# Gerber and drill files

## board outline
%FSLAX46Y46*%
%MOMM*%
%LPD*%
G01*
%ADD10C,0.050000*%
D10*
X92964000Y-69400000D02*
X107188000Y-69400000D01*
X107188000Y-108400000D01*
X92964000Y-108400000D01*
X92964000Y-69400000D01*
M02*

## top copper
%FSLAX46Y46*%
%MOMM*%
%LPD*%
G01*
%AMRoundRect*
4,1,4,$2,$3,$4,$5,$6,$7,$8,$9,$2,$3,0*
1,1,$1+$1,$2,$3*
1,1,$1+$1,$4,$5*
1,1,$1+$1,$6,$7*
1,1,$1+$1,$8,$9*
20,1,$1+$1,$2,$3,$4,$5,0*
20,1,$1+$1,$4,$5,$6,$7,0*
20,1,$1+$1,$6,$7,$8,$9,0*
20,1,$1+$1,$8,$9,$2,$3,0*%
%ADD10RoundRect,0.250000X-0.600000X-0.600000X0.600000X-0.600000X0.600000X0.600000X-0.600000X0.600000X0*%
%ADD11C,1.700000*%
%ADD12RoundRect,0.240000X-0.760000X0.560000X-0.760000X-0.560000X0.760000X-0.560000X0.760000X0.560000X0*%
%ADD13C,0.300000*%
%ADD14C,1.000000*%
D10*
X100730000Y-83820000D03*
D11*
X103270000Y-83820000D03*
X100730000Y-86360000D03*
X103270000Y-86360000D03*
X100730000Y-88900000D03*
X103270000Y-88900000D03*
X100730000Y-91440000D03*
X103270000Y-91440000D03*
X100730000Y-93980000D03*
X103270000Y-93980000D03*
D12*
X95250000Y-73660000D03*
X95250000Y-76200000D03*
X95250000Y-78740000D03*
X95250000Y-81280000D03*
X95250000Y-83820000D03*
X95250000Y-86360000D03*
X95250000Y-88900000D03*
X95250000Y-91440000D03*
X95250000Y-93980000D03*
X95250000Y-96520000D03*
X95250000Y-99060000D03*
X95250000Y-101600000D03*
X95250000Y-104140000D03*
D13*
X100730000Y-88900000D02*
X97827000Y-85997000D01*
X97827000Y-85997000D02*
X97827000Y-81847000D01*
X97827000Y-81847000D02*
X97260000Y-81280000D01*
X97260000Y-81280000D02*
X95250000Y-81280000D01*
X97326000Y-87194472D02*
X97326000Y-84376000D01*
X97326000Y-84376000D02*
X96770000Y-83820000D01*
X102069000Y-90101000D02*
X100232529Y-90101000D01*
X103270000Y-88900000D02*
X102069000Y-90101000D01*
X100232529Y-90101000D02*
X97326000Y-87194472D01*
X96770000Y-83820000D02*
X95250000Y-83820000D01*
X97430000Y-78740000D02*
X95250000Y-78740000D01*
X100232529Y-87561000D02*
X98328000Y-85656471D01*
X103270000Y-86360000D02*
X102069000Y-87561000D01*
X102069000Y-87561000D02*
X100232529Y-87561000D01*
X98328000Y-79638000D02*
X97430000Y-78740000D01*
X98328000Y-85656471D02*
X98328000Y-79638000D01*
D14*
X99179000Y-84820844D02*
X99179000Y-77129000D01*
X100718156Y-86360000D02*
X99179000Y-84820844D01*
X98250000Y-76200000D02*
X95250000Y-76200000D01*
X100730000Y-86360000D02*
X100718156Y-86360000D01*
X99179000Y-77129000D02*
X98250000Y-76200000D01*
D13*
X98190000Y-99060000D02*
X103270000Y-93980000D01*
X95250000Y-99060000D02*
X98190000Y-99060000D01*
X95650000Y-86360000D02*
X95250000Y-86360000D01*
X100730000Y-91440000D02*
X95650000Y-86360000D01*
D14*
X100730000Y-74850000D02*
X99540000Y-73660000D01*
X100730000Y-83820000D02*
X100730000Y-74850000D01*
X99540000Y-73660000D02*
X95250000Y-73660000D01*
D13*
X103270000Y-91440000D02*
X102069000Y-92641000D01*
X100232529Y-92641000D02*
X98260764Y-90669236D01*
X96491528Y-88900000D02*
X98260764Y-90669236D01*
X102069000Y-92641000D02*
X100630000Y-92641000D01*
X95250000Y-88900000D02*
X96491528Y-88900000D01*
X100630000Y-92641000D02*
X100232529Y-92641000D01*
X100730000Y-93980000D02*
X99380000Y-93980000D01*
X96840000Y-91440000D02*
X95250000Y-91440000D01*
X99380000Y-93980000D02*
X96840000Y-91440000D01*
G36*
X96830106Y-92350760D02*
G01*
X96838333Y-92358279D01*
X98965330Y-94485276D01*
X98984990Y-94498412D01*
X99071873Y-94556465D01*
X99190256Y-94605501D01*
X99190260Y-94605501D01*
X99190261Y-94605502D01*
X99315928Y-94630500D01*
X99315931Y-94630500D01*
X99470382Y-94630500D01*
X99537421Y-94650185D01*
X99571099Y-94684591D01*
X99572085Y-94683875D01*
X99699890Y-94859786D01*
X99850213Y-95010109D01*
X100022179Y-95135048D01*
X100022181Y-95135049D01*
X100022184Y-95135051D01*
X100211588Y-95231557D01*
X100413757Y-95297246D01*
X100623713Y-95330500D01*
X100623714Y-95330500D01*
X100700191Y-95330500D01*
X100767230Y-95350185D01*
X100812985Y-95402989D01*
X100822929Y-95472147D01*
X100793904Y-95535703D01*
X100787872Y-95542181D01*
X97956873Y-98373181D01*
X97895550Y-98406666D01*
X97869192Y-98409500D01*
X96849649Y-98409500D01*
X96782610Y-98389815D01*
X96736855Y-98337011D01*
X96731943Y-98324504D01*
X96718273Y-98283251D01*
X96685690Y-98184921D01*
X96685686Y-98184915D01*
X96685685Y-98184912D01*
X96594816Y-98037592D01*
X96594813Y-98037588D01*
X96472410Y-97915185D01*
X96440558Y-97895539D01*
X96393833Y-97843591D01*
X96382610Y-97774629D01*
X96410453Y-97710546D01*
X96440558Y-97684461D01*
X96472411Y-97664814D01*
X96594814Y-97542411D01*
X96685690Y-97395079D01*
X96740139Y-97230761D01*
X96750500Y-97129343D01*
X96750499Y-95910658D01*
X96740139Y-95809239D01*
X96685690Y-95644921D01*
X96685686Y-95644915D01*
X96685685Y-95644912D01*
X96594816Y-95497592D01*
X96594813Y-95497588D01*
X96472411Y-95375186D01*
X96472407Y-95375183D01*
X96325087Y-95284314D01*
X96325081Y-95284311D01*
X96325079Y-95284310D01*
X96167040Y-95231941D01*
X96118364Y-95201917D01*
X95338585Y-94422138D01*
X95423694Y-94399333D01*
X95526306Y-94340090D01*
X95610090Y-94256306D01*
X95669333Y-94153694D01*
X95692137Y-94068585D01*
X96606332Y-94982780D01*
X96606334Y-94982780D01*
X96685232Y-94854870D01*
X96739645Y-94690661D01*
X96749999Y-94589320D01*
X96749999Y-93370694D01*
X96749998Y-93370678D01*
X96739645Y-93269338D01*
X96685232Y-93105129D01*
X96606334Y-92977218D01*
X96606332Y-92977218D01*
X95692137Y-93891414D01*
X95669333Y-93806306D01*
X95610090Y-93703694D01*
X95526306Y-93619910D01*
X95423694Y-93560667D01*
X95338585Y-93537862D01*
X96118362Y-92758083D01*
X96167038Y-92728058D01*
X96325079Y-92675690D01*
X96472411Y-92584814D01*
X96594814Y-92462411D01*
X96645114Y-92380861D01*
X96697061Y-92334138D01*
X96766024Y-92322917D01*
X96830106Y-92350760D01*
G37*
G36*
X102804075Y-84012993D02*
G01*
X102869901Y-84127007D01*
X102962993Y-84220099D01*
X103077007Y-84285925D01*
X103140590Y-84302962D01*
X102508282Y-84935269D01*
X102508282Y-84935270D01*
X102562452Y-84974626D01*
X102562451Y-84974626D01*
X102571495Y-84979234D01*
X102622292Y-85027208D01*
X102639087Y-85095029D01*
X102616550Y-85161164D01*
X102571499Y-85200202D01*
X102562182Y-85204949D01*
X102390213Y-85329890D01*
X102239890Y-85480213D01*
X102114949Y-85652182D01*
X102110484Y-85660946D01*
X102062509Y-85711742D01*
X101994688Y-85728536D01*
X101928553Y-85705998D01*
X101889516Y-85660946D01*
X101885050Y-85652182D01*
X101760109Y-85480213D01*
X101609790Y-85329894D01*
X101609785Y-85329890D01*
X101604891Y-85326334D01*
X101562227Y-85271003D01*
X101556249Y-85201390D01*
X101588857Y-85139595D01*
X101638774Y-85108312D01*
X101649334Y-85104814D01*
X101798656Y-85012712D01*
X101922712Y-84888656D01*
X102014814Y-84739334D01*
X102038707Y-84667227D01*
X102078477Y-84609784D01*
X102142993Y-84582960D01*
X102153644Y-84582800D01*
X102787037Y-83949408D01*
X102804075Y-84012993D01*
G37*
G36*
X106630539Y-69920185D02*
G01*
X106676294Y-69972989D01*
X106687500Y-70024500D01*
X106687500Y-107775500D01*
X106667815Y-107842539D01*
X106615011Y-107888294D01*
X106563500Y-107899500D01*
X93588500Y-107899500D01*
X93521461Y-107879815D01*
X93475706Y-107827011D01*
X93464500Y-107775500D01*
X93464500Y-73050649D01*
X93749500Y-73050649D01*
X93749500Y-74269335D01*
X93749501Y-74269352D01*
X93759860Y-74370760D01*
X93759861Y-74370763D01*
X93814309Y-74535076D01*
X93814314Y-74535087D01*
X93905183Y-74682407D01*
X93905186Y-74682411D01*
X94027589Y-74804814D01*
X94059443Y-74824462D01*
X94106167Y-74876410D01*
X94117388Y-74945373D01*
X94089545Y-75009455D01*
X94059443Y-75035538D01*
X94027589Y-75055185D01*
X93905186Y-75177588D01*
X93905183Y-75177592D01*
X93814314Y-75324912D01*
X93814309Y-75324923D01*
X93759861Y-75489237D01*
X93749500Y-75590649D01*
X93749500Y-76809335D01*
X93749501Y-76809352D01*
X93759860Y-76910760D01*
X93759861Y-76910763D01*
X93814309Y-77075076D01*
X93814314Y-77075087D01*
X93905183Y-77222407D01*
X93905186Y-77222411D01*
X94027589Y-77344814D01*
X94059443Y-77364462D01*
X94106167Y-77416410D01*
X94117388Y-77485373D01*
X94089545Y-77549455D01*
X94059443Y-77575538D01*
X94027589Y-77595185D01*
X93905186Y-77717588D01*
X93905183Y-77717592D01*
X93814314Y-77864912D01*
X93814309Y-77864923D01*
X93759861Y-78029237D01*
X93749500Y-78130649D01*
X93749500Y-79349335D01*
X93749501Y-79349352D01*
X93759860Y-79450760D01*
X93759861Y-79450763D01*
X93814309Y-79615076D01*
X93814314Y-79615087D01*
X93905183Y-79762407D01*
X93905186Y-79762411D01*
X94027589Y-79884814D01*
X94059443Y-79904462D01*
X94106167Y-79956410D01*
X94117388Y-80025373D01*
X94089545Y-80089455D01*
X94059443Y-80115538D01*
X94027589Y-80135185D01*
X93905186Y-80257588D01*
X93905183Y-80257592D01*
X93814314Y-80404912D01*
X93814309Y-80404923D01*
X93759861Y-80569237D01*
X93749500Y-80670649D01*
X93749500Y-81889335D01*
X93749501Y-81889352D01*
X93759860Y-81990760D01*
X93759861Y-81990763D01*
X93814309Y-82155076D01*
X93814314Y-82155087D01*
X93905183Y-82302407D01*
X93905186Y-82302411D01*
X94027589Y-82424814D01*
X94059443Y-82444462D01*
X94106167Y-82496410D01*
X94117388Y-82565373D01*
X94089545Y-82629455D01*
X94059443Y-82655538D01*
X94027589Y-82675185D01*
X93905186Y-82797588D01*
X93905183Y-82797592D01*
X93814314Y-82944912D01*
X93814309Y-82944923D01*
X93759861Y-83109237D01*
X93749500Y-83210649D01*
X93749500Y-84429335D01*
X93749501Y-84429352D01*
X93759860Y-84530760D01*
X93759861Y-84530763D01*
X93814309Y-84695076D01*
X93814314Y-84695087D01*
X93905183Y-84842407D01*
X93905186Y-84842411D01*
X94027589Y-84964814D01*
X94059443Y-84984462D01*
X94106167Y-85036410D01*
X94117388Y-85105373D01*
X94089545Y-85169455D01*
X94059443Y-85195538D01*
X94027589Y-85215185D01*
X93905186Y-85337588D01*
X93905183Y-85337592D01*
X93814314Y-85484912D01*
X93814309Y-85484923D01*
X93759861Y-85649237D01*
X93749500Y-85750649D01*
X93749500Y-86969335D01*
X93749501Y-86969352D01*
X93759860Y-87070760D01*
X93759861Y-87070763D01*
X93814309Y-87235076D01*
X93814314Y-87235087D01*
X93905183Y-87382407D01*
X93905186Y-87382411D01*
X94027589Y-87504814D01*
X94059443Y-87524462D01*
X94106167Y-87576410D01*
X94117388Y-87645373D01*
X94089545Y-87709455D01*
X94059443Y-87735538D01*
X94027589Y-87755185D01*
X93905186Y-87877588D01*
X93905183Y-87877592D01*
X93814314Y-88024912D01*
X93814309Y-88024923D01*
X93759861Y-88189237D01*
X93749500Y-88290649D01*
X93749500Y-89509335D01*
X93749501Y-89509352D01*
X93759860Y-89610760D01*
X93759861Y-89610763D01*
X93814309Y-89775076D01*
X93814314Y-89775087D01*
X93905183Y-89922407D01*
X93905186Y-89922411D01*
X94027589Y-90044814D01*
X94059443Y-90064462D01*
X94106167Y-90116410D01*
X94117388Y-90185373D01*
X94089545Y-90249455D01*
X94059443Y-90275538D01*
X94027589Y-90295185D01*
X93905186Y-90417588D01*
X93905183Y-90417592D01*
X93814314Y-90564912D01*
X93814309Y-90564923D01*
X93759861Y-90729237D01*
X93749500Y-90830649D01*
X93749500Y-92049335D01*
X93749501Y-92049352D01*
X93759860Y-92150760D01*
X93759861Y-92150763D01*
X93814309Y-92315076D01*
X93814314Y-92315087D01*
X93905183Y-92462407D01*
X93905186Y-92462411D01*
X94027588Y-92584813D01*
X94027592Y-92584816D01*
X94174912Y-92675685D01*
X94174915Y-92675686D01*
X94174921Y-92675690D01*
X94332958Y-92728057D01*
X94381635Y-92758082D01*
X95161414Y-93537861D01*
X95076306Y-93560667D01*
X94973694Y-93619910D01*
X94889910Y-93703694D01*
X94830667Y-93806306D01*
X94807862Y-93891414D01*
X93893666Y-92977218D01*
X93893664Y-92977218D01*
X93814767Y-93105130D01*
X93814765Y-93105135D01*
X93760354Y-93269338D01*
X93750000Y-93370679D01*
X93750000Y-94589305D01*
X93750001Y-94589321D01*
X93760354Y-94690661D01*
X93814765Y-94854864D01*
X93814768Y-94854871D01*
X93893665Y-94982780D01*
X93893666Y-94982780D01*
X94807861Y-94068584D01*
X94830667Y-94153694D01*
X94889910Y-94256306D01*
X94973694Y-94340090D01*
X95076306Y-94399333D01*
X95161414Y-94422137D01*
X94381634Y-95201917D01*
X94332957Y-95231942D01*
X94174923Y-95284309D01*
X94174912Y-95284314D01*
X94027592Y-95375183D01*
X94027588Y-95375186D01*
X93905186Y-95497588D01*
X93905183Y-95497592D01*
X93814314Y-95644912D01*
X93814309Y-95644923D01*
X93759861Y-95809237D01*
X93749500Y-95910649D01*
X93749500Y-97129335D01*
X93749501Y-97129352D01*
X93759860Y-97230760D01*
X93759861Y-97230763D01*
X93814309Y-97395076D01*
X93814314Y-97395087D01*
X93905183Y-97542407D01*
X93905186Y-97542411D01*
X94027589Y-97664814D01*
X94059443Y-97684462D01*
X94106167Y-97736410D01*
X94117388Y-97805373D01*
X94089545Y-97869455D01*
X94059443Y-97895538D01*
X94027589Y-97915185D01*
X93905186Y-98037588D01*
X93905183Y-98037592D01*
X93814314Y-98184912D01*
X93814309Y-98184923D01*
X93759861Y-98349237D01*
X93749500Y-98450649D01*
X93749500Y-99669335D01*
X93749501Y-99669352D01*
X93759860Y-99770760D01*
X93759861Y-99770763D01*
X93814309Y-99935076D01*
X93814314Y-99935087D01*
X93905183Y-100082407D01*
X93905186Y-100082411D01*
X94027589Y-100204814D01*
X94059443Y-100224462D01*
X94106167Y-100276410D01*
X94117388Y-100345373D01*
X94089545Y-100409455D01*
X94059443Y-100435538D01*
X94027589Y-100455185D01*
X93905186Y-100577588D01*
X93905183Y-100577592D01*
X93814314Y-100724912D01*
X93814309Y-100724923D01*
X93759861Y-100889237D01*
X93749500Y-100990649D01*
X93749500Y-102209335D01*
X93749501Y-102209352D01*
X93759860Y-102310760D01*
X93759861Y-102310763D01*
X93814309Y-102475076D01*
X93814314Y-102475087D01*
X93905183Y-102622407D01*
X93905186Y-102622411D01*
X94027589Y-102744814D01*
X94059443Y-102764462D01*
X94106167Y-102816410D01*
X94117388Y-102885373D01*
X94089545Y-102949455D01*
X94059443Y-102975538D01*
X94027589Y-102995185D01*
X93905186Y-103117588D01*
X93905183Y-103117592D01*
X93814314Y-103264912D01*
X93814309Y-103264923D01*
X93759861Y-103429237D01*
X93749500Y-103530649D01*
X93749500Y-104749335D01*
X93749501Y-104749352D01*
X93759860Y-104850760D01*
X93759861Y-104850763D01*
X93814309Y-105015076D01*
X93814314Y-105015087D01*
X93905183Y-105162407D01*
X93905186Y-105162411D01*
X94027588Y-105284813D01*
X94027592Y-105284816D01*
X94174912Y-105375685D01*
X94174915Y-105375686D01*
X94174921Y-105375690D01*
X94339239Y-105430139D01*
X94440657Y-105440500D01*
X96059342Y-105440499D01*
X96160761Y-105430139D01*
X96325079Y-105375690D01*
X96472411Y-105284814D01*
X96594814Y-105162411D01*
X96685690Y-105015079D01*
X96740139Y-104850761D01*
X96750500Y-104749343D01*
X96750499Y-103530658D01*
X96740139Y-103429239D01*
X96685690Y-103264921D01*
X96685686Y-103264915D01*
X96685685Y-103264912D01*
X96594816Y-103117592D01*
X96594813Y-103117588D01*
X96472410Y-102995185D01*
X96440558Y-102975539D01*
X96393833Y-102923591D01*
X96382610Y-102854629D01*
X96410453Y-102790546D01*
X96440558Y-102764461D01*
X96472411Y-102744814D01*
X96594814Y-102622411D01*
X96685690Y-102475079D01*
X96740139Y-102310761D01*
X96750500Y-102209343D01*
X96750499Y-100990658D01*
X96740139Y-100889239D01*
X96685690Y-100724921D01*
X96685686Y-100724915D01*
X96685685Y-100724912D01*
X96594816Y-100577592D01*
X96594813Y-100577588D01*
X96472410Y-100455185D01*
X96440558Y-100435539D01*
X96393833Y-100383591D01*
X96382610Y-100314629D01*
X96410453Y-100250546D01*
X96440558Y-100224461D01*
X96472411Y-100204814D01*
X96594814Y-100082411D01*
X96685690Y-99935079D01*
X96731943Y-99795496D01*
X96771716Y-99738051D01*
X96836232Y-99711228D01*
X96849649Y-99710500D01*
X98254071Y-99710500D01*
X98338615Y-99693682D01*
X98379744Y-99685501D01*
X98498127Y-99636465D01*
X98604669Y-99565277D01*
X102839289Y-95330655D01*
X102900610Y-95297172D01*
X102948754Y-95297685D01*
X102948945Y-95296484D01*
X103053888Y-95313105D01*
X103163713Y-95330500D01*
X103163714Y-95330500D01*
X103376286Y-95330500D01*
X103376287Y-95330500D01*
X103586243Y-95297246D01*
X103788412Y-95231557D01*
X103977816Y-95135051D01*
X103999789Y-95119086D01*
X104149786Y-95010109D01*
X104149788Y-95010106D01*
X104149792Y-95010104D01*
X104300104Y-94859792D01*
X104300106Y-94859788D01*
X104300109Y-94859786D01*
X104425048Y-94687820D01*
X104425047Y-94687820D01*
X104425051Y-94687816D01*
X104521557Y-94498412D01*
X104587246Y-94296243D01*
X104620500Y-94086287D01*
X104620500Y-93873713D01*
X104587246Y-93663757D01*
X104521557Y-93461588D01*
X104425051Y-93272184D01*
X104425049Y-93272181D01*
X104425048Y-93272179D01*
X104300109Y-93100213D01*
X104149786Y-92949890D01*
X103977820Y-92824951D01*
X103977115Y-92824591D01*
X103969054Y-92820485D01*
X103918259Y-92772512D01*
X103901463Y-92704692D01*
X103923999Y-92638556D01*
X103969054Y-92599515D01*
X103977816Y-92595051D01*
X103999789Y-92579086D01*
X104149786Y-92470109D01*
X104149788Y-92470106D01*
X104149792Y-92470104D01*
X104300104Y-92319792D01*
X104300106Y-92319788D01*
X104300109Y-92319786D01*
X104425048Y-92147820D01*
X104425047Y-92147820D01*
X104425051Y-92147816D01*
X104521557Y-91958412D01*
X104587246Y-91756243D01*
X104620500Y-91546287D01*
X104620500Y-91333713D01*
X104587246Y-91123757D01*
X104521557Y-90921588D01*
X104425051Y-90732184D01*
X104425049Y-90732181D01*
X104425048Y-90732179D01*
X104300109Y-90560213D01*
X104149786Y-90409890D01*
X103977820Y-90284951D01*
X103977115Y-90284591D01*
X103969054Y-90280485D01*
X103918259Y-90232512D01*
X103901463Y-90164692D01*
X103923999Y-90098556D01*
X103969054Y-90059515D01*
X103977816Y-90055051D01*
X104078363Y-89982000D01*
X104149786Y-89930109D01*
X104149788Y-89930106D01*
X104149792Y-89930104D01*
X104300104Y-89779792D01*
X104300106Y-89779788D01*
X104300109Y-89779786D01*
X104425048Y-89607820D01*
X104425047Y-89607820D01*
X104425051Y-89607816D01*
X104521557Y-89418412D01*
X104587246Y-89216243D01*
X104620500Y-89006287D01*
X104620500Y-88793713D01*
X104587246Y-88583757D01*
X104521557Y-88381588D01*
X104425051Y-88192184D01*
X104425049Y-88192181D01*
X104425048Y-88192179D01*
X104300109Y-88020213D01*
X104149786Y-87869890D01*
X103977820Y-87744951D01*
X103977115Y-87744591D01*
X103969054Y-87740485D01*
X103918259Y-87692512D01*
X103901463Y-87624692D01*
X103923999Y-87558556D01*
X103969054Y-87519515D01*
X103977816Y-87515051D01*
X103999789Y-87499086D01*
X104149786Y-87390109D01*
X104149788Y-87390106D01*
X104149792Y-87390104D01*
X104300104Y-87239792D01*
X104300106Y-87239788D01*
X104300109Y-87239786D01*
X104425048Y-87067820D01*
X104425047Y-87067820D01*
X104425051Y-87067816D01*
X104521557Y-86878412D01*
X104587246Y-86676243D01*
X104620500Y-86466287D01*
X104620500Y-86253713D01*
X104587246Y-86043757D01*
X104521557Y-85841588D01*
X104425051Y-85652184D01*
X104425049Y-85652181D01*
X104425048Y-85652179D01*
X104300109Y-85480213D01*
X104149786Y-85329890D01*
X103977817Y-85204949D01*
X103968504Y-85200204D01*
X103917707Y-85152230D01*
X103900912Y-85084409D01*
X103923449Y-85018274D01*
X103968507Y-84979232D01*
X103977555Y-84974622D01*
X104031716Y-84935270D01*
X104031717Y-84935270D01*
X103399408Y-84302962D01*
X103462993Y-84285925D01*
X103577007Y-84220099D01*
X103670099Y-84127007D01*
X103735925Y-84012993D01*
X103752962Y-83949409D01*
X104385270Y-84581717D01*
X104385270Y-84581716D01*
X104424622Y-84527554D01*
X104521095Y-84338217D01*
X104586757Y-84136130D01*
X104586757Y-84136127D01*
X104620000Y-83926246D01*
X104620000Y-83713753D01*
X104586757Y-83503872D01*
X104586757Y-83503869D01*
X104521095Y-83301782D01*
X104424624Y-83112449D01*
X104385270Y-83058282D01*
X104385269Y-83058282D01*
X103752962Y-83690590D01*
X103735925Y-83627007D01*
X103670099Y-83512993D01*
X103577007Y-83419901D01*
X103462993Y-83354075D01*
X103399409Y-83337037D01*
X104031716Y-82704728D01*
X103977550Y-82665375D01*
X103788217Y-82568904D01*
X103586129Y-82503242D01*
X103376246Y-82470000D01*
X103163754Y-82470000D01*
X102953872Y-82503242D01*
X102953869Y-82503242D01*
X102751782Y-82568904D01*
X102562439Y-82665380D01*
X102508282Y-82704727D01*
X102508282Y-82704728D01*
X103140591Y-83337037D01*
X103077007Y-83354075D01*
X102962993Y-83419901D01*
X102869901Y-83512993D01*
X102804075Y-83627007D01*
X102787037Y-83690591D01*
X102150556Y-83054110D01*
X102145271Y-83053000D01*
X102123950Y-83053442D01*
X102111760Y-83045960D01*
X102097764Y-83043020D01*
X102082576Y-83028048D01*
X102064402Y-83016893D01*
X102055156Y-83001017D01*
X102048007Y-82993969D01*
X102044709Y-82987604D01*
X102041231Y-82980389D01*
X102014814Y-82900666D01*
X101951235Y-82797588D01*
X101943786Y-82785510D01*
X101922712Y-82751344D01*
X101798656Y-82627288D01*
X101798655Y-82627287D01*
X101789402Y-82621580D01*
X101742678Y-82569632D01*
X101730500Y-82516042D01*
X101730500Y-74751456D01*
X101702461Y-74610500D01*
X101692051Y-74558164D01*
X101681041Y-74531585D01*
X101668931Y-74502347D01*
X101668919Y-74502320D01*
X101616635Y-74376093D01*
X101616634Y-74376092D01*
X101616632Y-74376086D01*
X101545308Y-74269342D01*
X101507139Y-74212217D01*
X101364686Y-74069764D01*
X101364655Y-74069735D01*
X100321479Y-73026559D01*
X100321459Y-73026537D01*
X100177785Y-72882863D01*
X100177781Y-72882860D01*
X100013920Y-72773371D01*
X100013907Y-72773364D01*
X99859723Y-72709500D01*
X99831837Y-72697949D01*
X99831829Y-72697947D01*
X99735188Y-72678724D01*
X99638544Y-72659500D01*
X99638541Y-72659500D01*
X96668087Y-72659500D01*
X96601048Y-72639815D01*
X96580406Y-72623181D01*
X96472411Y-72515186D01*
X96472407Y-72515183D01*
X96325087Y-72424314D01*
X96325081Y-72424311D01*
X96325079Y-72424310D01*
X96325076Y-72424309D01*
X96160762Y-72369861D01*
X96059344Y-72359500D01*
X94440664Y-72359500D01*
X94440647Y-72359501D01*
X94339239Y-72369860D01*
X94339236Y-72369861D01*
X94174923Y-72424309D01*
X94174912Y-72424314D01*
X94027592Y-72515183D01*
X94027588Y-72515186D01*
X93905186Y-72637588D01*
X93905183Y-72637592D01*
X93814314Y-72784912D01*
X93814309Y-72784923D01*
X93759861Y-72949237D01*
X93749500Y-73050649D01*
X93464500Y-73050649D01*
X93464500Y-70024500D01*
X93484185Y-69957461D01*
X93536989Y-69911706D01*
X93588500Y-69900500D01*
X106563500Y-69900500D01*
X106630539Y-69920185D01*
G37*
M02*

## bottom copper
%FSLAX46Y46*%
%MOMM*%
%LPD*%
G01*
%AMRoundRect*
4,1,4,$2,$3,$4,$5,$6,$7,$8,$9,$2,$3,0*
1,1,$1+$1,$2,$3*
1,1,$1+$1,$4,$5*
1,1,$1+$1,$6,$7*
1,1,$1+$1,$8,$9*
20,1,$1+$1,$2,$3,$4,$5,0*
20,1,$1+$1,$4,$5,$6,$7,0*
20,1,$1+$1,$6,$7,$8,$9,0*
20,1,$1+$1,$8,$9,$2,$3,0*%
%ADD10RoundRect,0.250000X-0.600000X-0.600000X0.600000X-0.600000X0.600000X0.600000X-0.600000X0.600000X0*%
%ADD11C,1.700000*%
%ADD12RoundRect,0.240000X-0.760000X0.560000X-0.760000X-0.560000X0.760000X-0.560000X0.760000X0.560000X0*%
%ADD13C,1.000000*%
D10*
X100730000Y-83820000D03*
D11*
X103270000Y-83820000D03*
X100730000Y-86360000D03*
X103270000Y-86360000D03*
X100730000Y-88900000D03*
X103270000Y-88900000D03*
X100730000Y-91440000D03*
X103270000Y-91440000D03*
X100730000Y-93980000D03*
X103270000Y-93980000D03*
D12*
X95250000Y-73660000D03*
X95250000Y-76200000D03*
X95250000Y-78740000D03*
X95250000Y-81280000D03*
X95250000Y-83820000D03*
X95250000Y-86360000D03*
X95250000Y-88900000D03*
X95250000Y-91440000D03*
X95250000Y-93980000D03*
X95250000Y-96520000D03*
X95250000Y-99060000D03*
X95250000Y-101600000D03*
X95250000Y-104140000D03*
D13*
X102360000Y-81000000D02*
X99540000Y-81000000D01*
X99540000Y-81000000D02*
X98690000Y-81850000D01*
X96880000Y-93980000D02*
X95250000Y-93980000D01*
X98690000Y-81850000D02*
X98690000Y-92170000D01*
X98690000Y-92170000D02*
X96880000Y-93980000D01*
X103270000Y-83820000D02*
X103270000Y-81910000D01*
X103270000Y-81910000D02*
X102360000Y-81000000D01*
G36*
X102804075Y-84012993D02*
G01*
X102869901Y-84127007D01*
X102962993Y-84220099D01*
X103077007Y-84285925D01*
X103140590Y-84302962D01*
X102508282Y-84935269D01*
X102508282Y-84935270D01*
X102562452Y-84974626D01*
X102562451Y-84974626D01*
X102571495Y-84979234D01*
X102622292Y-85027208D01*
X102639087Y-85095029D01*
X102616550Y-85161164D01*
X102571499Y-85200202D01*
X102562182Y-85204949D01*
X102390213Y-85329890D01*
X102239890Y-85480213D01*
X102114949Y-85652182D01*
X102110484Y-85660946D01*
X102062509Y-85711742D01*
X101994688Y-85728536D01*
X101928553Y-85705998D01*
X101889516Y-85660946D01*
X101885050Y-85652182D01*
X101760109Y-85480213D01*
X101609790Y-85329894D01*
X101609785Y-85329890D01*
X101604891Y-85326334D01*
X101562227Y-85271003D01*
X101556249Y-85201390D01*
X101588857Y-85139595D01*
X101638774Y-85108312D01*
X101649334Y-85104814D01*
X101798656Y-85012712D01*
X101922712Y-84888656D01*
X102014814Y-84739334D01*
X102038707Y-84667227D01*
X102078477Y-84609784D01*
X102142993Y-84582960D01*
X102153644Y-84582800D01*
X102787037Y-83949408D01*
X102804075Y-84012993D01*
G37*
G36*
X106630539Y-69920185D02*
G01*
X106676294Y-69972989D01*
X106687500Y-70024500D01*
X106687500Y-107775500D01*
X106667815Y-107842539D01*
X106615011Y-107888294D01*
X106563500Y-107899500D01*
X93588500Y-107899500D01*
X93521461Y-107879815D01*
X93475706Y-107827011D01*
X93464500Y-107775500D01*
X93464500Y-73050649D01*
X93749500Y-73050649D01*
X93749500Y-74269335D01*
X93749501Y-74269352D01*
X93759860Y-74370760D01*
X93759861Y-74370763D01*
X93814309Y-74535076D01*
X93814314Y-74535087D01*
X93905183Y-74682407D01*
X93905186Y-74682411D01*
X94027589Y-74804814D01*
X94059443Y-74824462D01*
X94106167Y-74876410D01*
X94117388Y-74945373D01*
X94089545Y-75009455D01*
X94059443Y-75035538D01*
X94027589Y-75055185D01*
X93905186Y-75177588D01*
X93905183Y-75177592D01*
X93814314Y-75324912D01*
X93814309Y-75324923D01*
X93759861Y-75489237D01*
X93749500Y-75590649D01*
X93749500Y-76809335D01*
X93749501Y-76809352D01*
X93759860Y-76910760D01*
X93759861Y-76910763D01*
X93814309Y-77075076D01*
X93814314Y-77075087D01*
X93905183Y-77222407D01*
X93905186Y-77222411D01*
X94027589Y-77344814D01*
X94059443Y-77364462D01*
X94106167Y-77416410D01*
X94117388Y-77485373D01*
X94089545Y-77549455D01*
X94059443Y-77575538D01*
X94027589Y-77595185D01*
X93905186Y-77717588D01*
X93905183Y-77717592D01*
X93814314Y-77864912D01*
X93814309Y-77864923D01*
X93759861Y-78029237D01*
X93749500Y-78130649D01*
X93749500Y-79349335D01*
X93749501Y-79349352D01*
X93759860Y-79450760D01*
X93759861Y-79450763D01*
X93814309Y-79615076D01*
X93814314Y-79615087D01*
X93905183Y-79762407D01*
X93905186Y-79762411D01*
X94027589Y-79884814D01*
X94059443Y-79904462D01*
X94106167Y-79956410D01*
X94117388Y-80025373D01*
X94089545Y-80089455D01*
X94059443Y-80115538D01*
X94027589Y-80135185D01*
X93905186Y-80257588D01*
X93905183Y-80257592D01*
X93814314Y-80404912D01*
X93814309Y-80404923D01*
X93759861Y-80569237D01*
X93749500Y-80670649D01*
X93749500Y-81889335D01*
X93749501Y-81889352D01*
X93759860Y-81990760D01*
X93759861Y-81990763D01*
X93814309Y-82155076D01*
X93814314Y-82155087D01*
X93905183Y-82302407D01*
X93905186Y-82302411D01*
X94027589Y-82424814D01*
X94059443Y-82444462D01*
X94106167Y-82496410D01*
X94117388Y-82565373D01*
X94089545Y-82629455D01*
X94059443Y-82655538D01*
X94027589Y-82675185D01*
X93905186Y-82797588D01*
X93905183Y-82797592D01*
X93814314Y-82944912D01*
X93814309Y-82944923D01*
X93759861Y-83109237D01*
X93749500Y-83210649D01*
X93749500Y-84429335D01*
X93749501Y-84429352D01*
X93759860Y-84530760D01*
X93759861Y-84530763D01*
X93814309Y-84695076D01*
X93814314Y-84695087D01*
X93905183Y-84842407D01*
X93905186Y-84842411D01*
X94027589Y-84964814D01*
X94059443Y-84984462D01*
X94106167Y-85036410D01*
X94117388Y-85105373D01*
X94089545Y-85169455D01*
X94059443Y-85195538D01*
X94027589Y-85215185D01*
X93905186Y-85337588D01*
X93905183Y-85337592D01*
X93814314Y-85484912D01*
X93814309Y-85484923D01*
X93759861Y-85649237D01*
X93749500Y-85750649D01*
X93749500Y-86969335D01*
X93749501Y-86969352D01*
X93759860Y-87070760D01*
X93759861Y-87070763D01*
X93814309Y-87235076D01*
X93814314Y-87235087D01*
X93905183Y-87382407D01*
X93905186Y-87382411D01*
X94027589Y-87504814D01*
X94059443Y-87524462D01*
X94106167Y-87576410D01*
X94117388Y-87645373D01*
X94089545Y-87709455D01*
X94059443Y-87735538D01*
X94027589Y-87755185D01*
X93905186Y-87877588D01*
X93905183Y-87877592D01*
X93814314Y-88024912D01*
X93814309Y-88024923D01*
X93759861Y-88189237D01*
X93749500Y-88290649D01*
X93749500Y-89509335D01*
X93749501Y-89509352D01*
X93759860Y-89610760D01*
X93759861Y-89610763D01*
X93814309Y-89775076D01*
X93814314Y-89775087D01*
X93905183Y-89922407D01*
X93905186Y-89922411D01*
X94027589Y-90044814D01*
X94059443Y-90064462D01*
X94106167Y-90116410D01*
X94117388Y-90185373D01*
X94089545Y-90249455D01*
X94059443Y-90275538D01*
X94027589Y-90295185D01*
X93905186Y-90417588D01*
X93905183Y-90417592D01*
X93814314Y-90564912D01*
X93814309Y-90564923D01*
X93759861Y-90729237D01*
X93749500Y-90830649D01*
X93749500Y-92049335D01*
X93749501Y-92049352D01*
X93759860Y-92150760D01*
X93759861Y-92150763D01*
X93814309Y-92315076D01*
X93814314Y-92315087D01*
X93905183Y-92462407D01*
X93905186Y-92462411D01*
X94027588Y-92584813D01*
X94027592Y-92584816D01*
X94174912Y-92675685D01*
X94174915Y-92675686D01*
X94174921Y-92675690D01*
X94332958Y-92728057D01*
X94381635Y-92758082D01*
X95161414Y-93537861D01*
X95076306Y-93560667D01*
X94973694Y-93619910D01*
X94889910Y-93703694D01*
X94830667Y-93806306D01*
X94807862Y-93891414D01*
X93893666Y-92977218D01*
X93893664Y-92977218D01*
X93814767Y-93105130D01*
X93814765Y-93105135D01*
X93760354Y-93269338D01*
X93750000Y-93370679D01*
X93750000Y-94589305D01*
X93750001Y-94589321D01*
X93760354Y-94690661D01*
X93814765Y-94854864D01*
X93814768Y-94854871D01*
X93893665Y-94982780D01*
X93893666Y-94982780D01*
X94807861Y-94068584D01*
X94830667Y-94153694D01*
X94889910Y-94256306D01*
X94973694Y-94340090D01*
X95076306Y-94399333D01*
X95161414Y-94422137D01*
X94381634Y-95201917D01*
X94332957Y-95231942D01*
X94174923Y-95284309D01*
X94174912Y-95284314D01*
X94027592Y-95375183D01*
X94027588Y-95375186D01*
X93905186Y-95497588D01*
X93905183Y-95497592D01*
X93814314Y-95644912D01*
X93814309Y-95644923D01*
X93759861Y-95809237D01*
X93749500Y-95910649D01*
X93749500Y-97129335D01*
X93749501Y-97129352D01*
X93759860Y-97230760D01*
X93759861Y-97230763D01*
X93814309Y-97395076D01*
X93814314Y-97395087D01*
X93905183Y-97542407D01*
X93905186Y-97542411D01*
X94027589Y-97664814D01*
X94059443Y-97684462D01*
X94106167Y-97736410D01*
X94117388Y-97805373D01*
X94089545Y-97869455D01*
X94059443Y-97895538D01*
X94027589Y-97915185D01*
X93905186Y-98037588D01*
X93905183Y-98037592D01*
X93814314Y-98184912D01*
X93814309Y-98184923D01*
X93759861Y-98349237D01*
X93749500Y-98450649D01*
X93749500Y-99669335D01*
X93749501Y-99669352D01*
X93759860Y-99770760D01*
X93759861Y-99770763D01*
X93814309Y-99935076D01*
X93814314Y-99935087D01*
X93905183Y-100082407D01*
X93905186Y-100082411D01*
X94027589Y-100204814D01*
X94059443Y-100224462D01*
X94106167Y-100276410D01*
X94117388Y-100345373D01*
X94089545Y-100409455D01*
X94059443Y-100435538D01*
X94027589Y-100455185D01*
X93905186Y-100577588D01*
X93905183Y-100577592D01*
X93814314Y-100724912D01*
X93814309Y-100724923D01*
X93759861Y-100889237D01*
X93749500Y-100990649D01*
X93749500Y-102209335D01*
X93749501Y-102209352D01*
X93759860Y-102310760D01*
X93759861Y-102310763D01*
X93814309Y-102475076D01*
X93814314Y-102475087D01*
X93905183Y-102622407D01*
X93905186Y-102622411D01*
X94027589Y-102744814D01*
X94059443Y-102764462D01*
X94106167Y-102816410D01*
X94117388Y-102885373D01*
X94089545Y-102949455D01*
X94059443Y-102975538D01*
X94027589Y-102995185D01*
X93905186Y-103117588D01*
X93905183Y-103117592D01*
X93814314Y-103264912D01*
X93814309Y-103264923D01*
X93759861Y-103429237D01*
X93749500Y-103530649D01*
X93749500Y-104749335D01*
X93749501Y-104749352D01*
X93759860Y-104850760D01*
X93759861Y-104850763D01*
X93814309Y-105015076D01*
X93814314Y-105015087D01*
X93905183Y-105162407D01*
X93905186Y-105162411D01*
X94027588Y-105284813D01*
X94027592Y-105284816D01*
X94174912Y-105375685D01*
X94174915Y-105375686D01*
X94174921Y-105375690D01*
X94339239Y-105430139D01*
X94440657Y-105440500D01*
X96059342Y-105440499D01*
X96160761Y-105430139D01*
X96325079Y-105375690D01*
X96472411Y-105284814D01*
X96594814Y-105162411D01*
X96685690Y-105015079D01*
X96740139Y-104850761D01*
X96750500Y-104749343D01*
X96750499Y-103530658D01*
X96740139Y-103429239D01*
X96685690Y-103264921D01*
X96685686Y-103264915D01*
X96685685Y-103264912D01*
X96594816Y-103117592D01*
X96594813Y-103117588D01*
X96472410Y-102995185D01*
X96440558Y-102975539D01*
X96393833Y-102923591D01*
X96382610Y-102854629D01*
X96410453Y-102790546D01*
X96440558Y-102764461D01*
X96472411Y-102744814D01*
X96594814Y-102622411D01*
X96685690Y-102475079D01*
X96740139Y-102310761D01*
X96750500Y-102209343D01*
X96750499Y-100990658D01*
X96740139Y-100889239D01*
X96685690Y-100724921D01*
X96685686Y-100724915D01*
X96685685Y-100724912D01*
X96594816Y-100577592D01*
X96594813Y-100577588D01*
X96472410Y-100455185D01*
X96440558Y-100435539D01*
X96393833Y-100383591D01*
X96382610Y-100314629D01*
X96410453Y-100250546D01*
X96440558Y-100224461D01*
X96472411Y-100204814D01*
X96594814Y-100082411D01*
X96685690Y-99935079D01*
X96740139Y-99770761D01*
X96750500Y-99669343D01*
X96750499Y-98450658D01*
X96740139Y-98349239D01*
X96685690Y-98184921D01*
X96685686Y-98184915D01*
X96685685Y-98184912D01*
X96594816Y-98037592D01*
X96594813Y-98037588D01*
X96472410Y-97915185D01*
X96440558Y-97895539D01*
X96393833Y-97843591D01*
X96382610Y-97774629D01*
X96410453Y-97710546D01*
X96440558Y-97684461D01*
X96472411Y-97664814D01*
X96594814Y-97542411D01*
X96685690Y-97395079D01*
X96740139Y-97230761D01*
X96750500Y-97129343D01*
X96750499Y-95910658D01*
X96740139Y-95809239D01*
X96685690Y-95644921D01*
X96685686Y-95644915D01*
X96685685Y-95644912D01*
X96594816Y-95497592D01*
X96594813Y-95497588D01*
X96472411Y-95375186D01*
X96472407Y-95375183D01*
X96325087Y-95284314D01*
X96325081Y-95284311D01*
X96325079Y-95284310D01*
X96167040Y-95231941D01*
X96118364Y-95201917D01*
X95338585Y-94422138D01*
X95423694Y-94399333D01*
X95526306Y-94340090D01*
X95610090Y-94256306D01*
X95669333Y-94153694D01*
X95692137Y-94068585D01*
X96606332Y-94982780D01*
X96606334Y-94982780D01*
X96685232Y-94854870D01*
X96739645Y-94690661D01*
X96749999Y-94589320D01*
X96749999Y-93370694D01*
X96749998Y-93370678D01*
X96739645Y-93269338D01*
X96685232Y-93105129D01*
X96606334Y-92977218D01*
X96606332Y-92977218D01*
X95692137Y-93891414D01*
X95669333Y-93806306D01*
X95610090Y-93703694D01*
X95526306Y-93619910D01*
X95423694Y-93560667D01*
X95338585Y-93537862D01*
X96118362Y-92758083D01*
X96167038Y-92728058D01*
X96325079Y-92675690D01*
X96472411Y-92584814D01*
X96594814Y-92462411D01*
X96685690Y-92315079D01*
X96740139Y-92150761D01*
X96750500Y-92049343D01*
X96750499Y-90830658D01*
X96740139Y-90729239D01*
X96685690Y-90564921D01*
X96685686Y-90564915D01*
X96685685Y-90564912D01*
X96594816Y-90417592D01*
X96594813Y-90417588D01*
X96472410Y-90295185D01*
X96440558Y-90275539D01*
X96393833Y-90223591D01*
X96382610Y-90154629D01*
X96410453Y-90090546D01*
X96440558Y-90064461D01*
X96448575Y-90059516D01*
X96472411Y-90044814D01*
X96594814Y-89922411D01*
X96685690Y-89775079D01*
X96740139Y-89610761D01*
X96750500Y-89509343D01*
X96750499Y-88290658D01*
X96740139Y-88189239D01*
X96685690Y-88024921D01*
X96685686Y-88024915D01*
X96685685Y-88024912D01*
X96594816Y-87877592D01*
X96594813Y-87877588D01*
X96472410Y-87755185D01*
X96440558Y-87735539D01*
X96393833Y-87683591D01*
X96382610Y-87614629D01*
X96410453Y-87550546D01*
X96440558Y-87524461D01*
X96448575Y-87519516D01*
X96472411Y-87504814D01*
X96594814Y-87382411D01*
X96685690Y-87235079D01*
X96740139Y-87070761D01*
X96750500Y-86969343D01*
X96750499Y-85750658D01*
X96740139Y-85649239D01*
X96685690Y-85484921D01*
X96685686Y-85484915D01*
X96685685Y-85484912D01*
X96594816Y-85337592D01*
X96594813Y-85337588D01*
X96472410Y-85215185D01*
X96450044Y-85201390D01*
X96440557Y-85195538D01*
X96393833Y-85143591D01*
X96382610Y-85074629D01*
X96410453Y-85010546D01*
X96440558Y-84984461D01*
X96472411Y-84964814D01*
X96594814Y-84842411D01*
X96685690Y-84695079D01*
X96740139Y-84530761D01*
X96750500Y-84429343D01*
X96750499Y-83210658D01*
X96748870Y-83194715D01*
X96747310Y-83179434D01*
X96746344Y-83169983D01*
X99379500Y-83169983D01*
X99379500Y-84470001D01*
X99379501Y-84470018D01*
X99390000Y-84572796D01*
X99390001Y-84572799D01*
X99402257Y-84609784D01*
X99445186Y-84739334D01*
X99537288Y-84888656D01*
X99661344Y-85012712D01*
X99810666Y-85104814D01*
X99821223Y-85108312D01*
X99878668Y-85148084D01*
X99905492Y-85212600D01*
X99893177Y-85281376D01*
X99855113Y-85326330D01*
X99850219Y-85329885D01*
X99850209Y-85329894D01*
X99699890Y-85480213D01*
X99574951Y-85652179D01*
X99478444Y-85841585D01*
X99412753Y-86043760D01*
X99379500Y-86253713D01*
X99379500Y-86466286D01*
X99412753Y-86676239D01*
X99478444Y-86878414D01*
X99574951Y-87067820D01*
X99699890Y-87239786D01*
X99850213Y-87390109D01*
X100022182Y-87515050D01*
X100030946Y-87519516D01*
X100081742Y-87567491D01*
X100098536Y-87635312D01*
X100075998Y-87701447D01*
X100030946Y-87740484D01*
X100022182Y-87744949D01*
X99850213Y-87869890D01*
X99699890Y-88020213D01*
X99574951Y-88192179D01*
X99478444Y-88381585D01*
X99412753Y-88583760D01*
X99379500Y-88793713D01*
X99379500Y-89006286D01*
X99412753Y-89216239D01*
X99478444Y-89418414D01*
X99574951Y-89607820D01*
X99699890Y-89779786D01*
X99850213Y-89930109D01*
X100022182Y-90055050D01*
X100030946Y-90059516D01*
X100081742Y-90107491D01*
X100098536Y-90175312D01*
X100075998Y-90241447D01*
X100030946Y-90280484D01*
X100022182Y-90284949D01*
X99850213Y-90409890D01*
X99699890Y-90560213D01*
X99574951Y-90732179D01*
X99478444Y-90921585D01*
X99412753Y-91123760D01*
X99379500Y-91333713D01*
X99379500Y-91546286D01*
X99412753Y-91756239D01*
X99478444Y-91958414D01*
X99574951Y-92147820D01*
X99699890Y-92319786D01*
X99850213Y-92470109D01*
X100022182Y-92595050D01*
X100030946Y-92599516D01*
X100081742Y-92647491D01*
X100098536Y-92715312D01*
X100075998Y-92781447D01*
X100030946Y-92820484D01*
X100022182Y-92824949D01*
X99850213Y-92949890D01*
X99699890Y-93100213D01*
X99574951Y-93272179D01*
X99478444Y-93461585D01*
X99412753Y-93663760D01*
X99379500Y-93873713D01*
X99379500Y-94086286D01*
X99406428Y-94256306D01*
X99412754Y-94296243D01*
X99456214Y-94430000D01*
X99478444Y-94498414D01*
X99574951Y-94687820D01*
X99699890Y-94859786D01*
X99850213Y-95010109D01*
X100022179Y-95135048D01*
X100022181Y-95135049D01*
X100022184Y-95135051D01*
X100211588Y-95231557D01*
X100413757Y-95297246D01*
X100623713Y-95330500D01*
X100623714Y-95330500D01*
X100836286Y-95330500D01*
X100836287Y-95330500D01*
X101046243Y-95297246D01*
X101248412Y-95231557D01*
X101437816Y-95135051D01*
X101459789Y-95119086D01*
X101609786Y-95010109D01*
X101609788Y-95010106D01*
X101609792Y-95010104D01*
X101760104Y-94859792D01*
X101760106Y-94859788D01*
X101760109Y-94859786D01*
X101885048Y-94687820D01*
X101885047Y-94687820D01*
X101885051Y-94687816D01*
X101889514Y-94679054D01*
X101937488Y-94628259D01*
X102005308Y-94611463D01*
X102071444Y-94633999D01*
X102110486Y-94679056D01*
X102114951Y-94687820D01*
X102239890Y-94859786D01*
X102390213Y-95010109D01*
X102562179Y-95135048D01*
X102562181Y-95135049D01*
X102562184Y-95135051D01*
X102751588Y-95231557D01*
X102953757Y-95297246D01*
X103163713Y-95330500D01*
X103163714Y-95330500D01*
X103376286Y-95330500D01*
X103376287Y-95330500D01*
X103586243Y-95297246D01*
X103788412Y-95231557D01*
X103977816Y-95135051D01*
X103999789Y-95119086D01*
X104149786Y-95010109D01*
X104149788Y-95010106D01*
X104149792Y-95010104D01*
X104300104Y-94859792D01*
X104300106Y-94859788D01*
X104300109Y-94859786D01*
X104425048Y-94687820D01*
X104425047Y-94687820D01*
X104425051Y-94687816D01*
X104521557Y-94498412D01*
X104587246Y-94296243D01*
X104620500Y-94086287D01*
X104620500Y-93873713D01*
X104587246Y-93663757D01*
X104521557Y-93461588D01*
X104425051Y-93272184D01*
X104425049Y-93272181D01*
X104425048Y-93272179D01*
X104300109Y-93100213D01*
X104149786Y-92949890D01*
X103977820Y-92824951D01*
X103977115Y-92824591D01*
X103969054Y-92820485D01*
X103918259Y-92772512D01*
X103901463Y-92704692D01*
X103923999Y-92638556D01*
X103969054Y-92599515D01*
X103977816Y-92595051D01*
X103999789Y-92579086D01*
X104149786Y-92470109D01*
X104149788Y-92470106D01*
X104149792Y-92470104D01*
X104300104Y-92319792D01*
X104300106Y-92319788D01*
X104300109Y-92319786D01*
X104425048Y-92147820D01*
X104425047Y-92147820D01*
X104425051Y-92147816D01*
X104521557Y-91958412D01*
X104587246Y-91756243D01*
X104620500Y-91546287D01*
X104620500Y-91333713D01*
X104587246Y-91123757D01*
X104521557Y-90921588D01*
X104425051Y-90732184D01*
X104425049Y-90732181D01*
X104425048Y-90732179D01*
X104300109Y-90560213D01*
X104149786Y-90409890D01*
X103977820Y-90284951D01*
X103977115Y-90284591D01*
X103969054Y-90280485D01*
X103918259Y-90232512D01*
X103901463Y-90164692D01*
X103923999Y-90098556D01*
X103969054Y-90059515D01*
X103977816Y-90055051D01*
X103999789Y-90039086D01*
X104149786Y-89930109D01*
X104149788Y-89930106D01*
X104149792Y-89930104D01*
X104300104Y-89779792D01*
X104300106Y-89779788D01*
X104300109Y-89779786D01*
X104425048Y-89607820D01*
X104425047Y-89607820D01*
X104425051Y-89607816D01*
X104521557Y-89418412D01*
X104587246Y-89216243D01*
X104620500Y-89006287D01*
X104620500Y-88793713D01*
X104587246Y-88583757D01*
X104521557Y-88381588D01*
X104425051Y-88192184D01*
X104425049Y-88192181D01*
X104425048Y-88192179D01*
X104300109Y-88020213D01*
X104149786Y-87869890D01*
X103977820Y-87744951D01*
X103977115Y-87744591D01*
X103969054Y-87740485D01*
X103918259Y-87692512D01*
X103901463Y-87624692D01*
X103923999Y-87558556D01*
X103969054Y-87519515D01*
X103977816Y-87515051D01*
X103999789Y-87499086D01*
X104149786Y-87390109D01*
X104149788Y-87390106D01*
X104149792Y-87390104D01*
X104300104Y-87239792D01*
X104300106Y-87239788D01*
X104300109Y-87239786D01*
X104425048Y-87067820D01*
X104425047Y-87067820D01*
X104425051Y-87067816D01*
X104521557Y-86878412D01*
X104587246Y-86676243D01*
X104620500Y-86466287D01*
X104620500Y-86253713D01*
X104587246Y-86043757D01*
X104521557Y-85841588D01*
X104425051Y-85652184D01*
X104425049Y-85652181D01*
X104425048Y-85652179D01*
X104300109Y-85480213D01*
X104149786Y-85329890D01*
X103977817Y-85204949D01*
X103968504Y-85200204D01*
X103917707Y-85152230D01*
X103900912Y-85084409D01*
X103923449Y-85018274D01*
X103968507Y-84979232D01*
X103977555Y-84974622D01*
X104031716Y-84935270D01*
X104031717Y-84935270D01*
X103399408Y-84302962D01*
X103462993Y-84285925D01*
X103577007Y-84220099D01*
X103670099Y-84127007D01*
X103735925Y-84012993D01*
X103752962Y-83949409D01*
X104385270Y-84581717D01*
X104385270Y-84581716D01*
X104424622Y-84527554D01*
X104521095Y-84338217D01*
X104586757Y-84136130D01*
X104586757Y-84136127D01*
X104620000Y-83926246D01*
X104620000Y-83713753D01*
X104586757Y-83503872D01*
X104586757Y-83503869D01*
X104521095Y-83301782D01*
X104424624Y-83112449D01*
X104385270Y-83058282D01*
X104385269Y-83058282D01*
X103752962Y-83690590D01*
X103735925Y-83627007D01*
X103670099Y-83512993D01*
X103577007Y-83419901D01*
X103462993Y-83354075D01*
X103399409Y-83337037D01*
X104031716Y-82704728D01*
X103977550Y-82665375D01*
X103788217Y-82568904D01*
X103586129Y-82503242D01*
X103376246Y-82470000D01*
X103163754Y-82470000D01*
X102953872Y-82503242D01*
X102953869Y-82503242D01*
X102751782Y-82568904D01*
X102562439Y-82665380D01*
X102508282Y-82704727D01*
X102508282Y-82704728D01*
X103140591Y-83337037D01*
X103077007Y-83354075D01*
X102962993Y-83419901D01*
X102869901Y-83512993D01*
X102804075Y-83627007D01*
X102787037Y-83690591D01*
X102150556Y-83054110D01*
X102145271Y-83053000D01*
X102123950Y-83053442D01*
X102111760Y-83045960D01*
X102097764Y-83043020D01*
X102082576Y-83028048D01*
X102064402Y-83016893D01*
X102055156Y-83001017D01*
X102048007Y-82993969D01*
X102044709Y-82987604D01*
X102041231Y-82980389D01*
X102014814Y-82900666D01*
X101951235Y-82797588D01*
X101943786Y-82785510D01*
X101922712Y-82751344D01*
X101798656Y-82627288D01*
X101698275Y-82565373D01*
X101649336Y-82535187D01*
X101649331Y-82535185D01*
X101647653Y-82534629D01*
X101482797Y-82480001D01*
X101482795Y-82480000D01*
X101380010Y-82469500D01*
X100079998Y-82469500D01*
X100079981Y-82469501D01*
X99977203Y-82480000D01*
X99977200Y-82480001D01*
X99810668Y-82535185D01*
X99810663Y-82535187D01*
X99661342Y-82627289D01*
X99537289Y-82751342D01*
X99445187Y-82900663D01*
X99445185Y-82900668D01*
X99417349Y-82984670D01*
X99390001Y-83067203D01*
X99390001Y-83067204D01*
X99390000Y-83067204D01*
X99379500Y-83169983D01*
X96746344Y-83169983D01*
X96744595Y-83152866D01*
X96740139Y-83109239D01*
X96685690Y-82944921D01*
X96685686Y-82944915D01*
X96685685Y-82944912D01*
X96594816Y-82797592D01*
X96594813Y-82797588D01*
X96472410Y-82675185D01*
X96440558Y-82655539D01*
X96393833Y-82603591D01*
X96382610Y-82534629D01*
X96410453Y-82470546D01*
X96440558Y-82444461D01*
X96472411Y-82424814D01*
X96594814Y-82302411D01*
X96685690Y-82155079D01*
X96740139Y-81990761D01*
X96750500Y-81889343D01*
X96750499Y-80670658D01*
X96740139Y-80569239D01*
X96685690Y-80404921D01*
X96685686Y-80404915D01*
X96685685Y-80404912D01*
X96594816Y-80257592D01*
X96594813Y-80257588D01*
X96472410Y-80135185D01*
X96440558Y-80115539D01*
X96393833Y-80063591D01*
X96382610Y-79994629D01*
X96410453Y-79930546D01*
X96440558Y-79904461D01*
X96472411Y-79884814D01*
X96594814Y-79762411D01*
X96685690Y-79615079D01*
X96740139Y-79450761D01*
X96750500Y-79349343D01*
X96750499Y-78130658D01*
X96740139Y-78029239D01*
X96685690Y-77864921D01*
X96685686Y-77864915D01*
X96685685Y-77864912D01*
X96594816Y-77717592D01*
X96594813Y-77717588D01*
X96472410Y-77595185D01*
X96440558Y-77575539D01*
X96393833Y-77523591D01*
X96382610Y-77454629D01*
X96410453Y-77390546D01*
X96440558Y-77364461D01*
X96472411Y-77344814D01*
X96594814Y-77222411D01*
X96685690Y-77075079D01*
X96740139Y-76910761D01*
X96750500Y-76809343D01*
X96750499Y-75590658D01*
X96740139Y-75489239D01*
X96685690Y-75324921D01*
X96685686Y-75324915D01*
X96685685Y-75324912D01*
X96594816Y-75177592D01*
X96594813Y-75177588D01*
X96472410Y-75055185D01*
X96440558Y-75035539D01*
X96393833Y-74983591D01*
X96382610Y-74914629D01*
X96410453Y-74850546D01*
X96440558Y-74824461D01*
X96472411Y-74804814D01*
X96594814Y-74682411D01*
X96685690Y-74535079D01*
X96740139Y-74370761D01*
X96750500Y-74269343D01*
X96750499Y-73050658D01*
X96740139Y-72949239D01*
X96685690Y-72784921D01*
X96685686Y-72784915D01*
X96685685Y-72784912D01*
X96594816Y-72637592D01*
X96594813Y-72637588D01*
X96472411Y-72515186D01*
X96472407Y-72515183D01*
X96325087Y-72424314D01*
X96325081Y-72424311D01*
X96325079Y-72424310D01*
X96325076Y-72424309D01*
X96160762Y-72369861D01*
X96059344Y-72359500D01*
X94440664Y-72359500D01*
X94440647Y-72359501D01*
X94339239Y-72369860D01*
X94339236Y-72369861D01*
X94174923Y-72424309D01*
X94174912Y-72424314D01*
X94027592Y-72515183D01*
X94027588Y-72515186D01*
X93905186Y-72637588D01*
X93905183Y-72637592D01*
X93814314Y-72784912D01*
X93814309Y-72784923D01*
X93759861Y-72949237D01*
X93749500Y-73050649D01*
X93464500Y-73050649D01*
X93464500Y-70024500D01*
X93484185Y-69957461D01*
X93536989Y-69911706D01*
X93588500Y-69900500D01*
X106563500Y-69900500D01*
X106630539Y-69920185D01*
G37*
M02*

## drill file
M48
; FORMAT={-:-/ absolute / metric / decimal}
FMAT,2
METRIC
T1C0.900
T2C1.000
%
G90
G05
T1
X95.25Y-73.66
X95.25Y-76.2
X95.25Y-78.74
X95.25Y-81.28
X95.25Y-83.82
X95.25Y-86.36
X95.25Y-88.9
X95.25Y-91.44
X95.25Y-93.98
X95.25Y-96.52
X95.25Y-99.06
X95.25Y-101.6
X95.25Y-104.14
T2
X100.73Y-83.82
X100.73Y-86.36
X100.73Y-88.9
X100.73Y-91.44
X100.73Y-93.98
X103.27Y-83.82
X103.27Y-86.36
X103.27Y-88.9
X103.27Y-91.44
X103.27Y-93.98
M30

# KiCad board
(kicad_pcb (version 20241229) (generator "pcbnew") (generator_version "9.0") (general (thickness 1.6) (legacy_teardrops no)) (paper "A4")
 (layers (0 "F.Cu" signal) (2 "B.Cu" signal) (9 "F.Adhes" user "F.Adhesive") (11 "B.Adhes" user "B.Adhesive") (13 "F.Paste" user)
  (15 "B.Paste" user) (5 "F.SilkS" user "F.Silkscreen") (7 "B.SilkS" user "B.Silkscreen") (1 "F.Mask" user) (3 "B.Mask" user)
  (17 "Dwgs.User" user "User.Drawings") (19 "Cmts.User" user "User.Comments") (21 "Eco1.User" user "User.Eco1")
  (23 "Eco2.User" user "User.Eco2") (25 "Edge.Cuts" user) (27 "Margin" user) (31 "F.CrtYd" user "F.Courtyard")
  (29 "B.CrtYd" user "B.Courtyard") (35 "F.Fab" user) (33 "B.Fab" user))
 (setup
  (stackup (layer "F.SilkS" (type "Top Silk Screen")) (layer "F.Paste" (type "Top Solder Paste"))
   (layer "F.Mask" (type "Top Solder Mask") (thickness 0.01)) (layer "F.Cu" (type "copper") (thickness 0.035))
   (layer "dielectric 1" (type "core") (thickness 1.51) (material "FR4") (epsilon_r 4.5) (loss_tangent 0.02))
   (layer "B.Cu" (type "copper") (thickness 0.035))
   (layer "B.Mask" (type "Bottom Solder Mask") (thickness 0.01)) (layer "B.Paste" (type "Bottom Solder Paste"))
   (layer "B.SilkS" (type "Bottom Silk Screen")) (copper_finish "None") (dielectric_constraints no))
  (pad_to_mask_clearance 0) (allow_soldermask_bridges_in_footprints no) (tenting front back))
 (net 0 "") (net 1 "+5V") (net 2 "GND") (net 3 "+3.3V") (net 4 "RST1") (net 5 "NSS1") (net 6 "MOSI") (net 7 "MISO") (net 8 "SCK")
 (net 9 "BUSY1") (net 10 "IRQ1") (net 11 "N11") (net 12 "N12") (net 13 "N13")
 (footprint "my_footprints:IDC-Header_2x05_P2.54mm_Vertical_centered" (layer "F.Cu") (at 102 88.9)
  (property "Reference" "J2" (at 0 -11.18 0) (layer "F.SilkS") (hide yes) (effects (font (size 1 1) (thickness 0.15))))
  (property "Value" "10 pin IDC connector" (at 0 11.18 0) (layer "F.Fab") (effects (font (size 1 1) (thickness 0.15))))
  (pad "1" thru_hole roundrect (at -1.27 -5.08) (size 1.7 1.7) (drill 1) (layers "*.Cu" "*.Mask") (remove_unused_layers no)
   (roundrect_rratio 0.147059) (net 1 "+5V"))
  (pad "2" thru_hole circle (at 1.27 -5.08) (size 1.7 1.7) (drill 1) (layers "*.Cu" "*.Mask") (remove_unused_layers no) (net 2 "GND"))
  (pad "3" thru_hole circle (at -1.27 -2.54) (size 1.7 1.7) (drill 1) (layers "*.Cu" "*.Mask") (remove_unused_layers no) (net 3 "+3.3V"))
  (pad "4" thru_hole circle (at 1.27 -2.54) (size 1.7 1.7) (drill 1) (layers "*.Cu" "*.Mask") (remove_unused_layers no) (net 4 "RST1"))
  (pad "5" thru_hole circle (at -1.27 0) (size 1.7 1.7) (drill 1) (layers "*.Cu" "*.Mask") (remove_unused_layers no) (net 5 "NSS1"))
  (pad "6" thru_hole circle (at 1.27 0) (size 1.7 1.7) (drill 1) (layers "*.Cu" "*.Mask") (remove_unused_layers no) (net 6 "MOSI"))
  (pad "7" thru_hole circle (at -1.27 2.54) (size 1.7 1.7) (drill 1) (layers "*.Cu" "*.Mask") (remove_unused_layers no) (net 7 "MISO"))
  (pad "8" thru_hole circle (at 1.27 2.54) (size 1.7 1.7) (drill 1) (layers "*.Cu" "*.Mask") (remove_unused_layers no) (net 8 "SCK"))
  (pad "9" thru_hole circle (at -1.27 5.08) (size 1.7 1.7) (drill 1) (layers "*.Cu" "*.Mask") (remove_unused_layers no) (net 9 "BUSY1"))
  (pad "10" thru_hole circle (at 1.27 5.08) (size 1.7 1.7) (drill 1) (layers "*.Cu" "*.Mask") (remove_unused_layers no) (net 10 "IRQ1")))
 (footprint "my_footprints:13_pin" (layer "F.Cu") (at 95.25 88.9 -90)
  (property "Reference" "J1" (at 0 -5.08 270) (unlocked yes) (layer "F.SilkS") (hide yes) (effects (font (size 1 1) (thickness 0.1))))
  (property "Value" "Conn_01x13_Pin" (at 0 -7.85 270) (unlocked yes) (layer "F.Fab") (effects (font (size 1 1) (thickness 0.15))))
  (pad "1" thru_hole roundrect (at -15.24 0 270) (size 1.6 2) (drill 0.9) (layers "*.Cu" "*.Mask") (remove_unused_layers no)
   (roundrect_rratio 0.15) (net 1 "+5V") (thermal_bridge_angle 45))
  (pad "2" thru_hole roundrect (at -12.7 0 270) (size 1.6 2) (drill 0.9) (layers "*.Cu" "*.Mask") (remove_unused_layers no)
   (roundrect_rratio 0.15) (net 3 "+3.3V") (thermal_bridge_angle 45))
  (pad "3" thru_hole roundrect (at -10.16 0 270) (size 1.6 2) (drill 0.9) (layers "*.Cu" "*.Mask") (remove_unused_layers no)
   (roundrect_rratio 0.15) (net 4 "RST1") (thermal_bridge_angle 45))
  (pad "4" thru_hole roundrect (at -7.62 0 270) (size 1.6 2) (drill 0.9) (layers "*.Cu" "*.Mask") (remove_unused_layers no)
   (roundrect_rratio 0.15) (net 5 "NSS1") (thermal_bridge_angle 45))
  (pad "5" thru_hole roundrect (at -5.08 0 270) (size 1.6 2) (drill 0.9) (layers "*.Cu" "*.Mask") (remove_unused_layers no)
   (roundrect_rratio 0.15) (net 6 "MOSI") (thermal_bridge_angle 45))
  (pad "6" thru_hole roundrect (at -2.54 0 270) (size 1.6 2) (drill 0.9) (layers "*.Cu" "*.Mask") (remove_unused_layers no)
   (roundrect_rratio 0.15) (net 7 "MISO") (thermal_bridge_angle 45))
  (pad "7" thru_hole roundrect (at 0 0 270) (size 1.6 2) (drill 0.9) (layers "*.Cu" "*.Mask") (remove_unused_layers no)
   (roundrect_rratio 0.15) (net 8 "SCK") (thermal_bridge_angle 45))
  (pad "8" thru_hole roundrect (at 2.54 0 270) (size 1.6 2) (drill 0.9) (layers "*.Cu" "*.Mask") (remove_unused_layers no)
   (roundrect_rratio 0.15) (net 9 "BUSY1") (thermal_bridge_angle 45))
  (pad "9" thru_hole roundrect (at 5.08 0 270) (size 1.6 2) (drill 0.9) (layers "*.Cu" "*.Mask") (remove_unused_layers no)
   (roundrect_rratio 0.15) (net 2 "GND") (thermal_bridge_angle 45))
  (pad "10" thru_hole roundrect (at 7.62 0 270) (size 1.6 2) (drill 0.9) (layers "*.Cu" "*.Mask") (remove_unused_layers no)
   (roundrect_rratio 0.15) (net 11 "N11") (thermal_bridge_angle 45))
  (pad "11" thru_hole roundrect (at 10.16 0 270) (size 1.6 2) (drill 0.9) (layers "*.Cu" "*.Mask") (remove_unused_layers no)
   (roundrect_rratio 0.15) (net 10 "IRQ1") (thermal_bridge_angle 45))
  (pad "12" thru_hole roundrect (at 12.7 0 270) (size 1.6 2) (drill 0.9) (layers "*.Cu" "*.Mask") (remove_unused_layers no)
   (roundrect_rratio 0.15) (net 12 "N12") (thermal_bridge_angle 45))
  (pad "13" thru_hole roundrect (at 15.24 0 270) (size 1.6 2) (drill 0.9) (layers "*.Cu" "*.Mask") (remove_unused_layers no)
   (roundrect_rratio 0.15) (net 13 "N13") (thermal_bridge_angle 45)))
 (gr_rect (start 92.964 69.4) (end 107.188 108.4) (stroke (width 0.05) (type solid)) (fill no) (layer "Edge.Cuts"))
 (segment (start 100.73 88.9) (end 97.827 85.997) (width 0.3) (layer "F.Cu") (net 5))
 (segment (start 97.827 85.997) (end 97.827 81.847) (width 0.3) (layer "F.Cu") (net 5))
 (segment (start 97.827 81.847) (end 97.26 81.28) (width 0.3) (layer "F.Cu") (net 5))
 (segment (start 97.26 81.28) (end 95.25 81.28) (width 0.3) (layer "F.Cu") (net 5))
 (segment (start 97.326 87.194472) (end 97.326 84.376) (width 0.3) (layer "F.Cu") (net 6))
 (segment (start 97.326 84.376) (end 96.77 83.82) (width 0.3) (layer "F.Cu") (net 6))
 (segment (start 102.069 90.101) (end 100.232529 90.101) (width 0.3) (layer "F.Cu") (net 6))
 (segment (start 103.27 88.9) (end 102.069 90.101) (width 0.3) (layer "F.Cu") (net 6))
 (segment (start 100.232529 90.101) (end 97.326 87.194472) (width 0.3) (layer "F.Cu") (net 6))
 (segment (start 96.77 83.82) (end 95.25 83.82) (width 0.3) (layer "F.Cu") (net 6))
 (segment (start 97.43 78.74) (end 95.25 78.74) (width 0.3) (layer "F.Cu") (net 4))
 (segment (start 100.232529 87.561) (end 98.328 85.656471) (width 0.3) (layer "F.Cu") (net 4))
 (segment (start 103.27 86.36) (end 102.069 87.561) (width 0.3) (layer "F.Cu") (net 4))
 (segment (start 102.069 87.561) (end 100.232529 87.561) (width 0.3) (layer "F.Cu") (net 4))
 (segment (start 98.328 79.638) (end 97.43 78.74) (width 0.3) (layer "F.Cu") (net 4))
 (segment (start 98.328 85.656471) (end 98.328 79.638) (width 0.3) (layer "F.Cu") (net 4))
 (segment (start 99.179 84.820844) (end 99.179 77.129) (width 1) (layer "F.Cu") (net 3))
 (segment (start 100.718156 86.36) (end 99.179 84.820844) (width 1) (layer "F.Cu") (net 3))
 (segment (start 98.25 76.2) (end 95.25 76.2) (width 1) (layer "F.Cu") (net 3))
 (segment (start 100.73 86.36) (end 100.718156 86.36) (width 1) (layer "F.Cu") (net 3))
 (segment (start 99.179 77.129) (end 98.25 76.2) (width 1) (layer "F.Cu") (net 3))
 (segment (start 98.19 99.06) (end 103.27 93.98) (width 0.3) (layer "F.Cu") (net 10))
 (segment (start 95.25 99.06) (end 98.19 99.06) (width 0.3) (layer "F.Cu") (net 10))
 (segment (start 95.65 86.36) (end 95.25 86.36) (width 0.3) (layer "F.Cu") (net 7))
 (segment (start 100.73 91.44) (end 95.65 86.36) (width 0.3) (layer "F.Cu") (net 7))
 (segment (start 100.73 74.85) (end 99.54 73.66) (width 1) (layer "F.Cu") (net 1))
 (segment (start 100.73 83.82) (end 100.73 74.85) (width 1) (layer "F.Cu") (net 1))
 (segment (start 99.54 73.66) (end 95.25 73.66) (width 1) (layer "F.Cu") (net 1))
 (segment (start 102.36 81) (end 99.54 81) (width 1) (layer "B.Cu") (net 2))
 (segment (start 99.54 81) (end 98.69 81.85) (width 1) (layer "B.Cu") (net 2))
 (segment (start 96.88 93.98) (end 95.25 93.98) (width 1) (layer "B.Cu") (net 2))
 (segment (start 98.69 81.85) (end 98.69 92.17) (width 1) (layer "B.Cu") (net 2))
 (segment (start 98.69 92.17) (end 96.88 93.98) (width 1) (layer "B.Cu") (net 2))
 (segment (start 103.27 83.82) (end 103.27 81.91) (width 1) (layer "B.Cu") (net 2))
 (segment (start 103.27 81.91) (end 102.36 81) (width 1) (layer "B.Cu") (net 2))
 (segment (start 103.27 91.44) (end 102.069 92.641) (width 0.3) (layer "F.Cu") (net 8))
 (segment (start 100.232529 92.641) (end 98.260764 90.669236) (width 0.3) (layer "F.Cu") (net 8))
 (segment (start 96.491528 88.9) (end 98.260764 90.669236) (width 0.3) (layer "F.Cu") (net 8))
 (segment (start 102.069 92.641) (end 100.63 92.641) (width 0.3) (layer "F.Cu") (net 8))
 (segment (start 95.25 88.9) (end 96.491528 88.9) (width 0.3) (layer "F.Cu") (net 8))
 (segment (start 100.63 92.641) (end 100.232529 92.641) (width 0.3) (layer "F.Cu") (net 8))
 (segment (start 100.73 93.98) (end 99.38 93.98) (width 0.3) (layer "F.Cu") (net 9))
 (segment (start 96.84 91.44) (end 95.25 91.44) (width 0.3) (layer "F.Cu") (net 9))
 (segment (start 99.38 93.98) (end 96.84 91.44) (width 0.3) (layer "F.Cu") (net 9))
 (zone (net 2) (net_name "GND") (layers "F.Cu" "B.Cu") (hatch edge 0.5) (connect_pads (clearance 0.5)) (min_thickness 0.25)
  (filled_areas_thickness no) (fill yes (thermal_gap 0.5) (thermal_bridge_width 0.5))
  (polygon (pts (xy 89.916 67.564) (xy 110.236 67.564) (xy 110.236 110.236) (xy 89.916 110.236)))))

